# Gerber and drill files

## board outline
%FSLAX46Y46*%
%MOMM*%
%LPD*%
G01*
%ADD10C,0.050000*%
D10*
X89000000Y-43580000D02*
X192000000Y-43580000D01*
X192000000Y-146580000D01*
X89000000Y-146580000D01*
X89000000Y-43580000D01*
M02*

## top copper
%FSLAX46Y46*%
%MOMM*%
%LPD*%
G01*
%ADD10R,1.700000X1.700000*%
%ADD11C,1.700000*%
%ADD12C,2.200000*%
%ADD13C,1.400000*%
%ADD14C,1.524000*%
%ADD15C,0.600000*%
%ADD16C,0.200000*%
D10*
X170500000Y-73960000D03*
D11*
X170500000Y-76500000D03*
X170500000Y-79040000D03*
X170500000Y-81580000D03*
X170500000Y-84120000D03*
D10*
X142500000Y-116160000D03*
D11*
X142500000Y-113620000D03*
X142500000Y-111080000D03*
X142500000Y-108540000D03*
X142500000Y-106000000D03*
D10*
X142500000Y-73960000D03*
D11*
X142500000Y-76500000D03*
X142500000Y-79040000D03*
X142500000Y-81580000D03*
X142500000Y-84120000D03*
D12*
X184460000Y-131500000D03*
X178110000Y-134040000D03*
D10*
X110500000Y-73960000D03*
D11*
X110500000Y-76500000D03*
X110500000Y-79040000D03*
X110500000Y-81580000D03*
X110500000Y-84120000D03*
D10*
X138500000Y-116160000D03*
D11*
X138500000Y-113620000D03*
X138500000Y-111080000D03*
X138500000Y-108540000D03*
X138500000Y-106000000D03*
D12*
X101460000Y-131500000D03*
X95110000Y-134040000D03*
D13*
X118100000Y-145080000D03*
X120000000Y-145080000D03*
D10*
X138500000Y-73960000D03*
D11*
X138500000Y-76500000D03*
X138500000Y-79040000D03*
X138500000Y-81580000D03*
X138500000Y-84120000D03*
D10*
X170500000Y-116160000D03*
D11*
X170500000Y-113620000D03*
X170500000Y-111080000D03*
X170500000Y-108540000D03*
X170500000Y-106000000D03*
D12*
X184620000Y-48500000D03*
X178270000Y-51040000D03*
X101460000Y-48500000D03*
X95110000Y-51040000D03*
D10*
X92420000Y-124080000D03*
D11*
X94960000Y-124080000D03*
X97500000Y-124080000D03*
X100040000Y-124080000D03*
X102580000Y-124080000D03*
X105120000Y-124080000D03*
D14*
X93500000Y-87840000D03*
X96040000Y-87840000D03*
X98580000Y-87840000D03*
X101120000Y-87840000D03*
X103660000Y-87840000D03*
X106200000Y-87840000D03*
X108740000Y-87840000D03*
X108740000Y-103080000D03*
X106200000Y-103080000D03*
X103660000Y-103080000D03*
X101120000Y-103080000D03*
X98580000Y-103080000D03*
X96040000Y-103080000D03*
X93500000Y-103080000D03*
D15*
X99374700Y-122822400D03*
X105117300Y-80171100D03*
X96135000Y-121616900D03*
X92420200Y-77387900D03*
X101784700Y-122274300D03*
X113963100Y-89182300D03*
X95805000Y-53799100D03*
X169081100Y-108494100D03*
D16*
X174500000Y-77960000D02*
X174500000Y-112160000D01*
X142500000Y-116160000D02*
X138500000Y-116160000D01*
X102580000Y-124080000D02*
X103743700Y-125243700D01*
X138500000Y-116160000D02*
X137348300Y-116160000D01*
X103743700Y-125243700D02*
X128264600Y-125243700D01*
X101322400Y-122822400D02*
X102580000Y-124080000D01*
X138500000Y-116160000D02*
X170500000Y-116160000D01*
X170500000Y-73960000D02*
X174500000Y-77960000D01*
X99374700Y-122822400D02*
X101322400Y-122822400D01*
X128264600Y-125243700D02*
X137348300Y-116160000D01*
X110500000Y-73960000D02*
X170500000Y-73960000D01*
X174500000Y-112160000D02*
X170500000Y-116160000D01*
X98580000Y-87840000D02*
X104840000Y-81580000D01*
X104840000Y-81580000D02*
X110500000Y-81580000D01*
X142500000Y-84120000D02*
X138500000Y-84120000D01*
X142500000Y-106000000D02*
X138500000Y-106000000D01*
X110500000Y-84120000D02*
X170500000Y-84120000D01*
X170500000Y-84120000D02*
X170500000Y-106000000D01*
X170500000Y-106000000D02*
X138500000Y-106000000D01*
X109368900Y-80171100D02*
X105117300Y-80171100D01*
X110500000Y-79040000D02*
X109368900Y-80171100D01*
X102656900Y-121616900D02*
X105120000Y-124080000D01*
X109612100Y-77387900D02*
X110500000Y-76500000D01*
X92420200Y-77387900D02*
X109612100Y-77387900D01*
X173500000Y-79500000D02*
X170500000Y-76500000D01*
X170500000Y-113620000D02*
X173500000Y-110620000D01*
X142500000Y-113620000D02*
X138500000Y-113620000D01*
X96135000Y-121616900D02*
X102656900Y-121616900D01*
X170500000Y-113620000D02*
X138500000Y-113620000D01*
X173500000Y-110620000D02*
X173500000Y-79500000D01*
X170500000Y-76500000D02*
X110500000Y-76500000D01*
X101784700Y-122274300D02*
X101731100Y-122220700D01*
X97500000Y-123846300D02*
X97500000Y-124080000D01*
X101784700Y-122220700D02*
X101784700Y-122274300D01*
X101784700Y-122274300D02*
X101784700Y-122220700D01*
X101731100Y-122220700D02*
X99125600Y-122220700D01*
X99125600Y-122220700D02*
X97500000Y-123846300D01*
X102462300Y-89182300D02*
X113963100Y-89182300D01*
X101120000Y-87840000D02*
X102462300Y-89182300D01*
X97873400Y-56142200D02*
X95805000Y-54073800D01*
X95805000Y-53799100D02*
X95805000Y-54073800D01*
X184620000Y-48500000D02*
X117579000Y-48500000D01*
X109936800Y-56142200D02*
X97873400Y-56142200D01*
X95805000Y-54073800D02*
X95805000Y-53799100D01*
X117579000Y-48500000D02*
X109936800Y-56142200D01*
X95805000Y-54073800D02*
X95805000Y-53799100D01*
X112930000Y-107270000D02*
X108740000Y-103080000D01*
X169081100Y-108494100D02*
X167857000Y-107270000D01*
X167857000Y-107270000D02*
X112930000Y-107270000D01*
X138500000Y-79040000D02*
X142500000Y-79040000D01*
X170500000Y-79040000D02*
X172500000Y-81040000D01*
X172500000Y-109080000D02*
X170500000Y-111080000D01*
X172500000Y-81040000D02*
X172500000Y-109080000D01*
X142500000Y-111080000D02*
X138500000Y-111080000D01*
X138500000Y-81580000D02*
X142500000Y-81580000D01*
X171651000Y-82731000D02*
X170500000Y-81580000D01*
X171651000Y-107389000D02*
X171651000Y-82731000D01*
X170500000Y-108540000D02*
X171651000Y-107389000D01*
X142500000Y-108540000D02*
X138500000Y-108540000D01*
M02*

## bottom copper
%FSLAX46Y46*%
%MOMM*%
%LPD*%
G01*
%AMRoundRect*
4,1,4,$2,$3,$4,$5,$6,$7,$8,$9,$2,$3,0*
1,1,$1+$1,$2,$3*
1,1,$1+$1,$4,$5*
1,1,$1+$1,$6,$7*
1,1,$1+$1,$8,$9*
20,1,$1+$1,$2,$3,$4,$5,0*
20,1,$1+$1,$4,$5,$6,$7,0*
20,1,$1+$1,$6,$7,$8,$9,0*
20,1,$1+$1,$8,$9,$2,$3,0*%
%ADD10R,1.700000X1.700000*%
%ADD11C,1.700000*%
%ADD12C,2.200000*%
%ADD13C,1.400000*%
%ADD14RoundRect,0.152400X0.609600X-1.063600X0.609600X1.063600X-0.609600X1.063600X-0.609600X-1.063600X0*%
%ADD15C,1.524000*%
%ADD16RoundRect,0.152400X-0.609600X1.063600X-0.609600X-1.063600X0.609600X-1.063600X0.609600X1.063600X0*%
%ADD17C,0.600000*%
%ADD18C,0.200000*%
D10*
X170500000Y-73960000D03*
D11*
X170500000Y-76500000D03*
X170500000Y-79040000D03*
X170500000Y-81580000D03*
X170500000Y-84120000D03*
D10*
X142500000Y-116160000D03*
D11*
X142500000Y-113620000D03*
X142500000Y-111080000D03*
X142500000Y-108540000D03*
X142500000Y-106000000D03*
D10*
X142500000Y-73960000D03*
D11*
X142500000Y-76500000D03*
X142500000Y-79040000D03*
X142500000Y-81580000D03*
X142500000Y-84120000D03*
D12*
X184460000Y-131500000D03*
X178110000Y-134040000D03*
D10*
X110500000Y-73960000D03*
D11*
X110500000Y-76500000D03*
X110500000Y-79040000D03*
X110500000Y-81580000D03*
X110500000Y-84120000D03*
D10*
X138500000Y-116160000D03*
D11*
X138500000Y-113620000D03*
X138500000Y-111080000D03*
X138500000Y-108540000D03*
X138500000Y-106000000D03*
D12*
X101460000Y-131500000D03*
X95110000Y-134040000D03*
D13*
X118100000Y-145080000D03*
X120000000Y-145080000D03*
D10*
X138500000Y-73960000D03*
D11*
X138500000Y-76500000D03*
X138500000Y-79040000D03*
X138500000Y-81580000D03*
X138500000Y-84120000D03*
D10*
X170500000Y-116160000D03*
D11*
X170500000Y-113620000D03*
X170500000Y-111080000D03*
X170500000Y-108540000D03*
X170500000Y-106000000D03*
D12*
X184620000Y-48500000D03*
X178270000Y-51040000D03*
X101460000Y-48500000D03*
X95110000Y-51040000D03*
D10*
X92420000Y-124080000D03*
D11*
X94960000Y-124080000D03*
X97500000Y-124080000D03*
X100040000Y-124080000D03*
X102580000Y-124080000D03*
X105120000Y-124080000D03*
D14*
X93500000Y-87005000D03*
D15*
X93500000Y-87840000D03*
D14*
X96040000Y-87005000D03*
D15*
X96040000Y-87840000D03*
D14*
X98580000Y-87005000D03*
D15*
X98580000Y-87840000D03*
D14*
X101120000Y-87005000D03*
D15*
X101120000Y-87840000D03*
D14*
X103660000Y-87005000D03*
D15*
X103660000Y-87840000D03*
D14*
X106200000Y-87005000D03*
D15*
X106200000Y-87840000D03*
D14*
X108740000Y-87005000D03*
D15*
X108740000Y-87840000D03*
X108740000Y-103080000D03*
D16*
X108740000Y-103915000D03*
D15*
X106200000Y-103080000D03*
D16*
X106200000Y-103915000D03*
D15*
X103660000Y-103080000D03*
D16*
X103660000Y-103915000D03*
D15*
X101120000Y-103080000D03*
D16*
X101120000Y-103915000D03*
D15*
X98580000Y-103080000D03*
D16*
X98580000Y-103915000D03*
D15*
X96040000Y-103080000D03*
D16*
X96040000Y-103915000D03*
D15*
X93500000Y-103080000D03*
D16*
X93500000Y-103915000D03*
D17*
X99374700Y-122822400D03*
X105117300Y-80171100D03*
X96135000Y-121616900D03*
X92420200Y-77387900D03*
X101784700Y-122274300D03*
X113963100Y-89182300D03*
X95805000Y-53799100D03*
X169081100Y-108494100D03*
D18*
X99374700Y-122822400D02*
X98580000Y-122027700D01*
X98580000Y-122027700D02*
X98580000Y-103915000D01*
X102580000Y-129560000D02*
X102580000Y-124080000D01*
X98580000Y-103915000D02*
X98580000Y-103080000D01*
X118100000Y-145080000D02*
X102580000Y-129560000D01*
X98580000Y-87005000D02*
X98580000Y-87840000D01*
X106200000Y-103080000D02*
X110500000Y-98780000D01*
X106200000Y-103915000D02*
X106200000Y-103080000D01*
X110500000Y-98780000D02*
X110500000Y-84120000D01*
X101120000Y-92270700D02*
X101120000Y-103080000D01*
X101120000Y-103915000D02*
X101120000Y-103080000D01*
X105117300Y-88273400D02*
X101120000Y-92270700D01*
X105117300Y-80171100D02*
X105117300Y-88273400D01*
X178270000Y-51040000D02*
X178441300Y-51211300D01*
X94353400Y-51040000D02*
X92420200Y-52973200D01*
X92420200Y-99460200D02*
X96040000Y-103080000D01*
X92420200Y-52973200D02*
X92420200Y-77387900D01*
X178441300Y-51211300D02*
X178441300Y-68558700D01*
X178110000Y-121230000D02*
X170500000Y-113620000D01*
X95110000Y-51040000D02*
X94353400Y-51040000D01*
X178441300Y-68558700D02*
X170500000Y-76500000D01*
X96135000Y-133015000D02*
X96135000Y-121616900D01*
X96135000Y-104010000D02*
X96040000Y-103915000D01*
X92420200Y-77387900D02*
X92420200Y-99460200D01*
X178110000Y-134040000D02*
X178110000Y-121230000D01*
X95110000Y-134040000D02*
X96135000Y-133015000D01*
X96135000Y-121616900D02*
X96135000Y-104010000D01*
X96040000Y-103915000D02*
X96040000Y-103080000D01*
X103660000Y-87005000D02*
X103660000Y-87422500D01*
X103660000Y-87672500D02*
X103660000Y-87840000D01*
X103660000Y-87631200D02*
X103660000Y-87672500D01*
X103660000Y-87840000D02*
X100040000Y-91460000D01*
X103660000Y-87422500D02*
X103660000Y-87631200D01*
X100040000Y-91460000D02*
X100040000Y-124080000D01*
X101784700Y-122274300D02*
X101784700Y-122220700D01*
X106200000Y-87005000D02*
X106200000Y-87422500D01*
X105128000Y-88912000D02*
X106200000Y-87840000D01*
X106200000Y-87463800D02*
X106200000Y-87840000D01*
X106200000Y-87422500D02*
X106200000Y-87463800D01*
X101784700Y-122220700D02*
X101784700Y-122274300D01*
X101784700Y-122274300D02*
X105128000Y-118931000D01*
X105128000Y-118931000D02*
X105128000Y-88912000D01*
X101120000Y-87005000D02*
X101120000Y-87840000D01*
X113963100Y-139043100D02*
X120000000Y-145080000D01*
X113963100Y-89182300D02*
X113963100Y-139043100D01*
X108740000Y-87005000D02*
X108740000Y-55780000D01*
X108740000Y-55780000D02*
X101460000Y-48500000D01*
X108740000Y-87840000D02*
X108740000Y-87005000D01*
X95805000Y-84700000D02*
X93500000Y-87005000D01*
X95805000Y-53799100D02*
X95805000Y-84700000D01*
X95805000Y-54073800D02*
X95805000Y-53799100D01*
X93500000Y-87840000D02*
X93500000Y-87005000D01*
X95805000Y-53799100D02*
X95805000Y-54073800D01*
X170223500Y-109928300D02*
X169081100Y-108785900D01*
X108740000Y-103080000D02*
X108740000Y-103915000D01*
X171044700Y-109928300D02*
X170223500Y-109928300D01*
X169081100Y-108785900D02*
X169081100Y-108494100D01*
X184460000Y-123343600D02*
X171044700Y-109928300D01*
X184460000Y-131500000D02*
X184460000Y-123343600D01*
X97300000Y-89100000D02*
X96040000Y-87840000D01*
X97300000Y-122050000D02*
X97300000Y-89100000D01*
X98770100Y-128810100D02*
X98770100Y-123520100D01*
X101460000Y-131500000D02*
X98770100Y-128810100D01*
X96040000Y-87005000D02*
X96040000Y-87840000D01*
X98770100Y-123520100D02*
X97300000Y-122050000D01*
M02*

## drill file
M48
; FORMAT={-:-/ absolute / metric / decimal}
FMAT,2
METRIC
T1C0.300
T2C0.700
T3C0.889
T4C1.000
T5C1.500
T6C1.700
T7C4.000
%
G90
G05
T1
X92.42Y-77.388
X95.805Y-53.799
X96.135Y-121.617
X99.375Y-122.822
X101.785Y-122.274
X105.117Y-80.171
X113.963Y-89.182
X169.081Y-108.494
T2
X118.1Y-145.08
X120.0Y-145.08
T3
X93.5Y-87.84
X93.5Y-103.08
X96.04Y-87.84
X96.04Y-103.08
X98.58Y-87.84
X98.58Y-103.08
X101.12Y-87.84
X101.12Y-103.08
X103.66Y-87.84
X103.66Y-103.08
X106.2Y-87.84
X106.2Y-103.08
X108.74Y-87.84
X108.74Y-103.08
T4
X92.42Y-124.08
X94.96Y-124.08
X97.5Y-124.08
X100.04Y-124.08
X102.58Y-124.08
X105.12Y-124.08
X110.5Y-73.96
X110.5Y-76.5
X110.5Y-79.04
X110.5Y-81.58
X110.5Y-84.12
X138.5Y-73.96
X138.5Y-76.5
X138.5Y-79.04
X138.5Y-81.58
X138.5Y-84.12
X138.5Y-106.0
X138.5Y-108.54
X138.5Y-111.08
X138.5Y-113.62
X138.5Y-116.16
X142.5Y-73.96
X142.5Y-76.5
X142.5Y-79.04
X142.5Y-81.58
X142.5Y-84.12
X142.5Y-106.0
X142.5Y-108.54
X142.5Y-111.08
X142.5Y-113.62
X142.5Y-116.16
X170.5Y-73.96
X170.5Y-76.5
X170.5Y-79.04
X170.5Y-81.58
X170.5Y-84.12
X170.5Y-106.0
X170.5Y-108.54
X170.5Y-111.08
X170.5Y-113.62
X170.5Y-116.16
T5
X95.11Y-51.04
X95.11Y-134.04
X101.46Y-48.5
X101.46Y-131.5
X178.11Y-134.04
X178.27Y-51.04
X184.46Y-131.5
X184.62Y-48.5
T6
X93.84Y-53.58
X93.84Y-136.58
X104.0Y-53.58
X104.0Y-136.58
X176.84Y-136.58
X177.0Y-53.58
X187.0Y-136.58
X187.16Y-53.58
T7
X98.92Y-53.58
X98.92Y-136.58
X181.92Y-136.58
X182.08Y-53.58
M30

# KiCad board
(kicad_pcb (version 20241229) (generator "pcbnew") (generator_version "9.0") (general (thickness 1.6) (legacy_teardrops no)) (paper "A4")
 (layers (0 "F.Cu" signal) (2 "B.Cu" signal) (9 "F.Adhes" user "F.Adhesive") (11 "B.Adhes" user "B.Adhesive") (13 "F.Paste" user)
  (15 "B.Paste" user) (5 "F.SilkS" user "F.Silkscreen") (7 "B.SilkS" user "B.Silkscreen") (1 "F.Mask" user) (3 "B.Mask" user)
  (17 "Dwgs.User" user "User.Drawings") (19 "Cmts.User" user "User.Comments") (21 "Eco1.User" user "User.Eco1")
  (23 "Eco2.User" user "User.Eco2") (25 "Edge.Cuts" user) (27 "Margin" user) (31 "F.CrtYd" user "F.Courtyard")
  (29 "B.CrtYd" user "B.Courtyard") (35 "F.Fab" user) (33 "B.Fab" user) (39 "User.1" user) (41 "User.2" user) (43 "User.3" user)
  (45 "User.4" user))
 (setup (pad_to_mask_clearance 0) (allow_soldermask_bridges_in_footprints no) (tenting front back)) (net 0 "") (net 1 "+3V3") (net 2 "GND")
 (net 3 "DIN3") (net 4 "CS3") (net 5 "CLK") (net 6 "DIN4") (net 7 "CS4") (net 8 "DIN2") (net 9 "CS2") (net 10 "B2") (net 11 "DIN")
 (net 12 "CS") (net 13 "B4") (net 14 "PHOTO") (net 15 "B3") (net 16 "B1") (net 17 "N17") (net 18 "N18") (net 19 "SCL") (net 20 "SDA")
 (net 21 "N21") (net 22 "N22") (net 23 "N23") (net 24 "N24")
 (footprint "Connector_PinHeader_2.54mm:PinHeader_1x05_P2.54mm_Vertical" (layer "F.Cu") (at 170.5 73.96)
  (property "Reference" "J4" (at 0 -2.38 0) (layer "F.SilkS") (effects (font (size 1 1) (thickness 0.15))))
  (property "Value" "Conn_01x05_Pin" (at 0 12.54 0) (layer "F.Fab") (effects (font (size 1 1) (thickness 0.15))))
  (pad "1" thru_hole rect (at 0 0) (size 1.7 1.7) (drill 1) (layers "*.Cu" "*.Mask") (remove_unused_layers no) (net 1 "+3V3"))
  (pad "2" thru_hole circle (at 0 2.54) (size 1.7 1.7) (drill 1) (layers "*.Cu" "*.Mask") (remove_unused_layers no) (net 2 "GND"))
  (pad "3" thru_hole circle (at 0 5.08) (size 1.7 1.7) (drill 1) (layers "*.Cu" "*.Mask") (remove_unused_layers no) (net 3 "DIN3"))
  (pad "4" thru_hole circle (at 0 7.62) (size 1.7 1.7) (drill 1) (layers "*.Cu" "*.Mask") (remove_unused_layers no) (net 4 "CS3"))
  (pad "5" thru_hole circle (at 0 10.16) (size 1.7 1.7) (drill 1) (layers "*.Cu" "*.Mask") (remove_unused_layers no) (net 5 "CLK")))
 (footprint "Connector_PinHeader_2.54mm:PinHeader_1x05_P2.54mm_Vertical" (layer "F.Cu") (at 142.5 116.16 180)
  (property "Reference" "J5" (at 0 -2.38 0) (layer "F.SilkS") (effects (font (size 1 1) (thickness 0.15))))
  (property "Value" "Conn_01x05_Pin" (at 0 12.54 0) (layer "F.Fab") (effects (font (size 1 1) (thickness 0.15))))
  (pad "1" thru_hole rect (at 0 0 180) (size 1.7 1.7) (drill 1) (layers "*.Cu" "*.Mask") (remove_unused_layers no) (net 1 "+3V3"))
  (pad "2" thru_hole circle (at 0 2.54 180) (size 1.7 1.7) (drill 1) (layers "*.Cu" "*.Mask") (remove_unused_layers no) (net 2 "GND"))
  (pad "3" thru_hole circle (at 0 5.08 180) (size 1.7 1.7) (drill 1) (layers "*.Cu" "*.Mask") (remove_unused_layers no) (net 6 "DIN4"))
  (pad "4" thru_hole circle (at 0 7.62 180) (size 1.7 1.7) (drill 1) (layers "*.Cu" "*.Mask") (remove_unused_layers no) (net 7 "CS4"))
  (pad "5" thru_hole circle (at 0 10.16 180) (size 1.7 1.7) (drill 1) (layers "*.Cu" "*.Mask") (remove_unused_layers no) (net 5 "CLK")))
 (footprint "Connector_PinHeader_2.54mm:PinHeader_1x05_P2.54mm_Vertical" (layer "F.Cu") (at 142.5 73.96)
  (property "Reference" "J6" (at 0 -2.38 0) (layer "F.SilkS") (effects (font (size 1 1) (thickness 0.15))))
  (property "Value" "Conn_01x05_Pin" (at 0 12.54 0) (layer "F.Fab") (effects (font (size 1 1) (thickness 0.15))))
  (pad "1" thru_hole rect (at 0 0) (size 1.7 1.7) (drill 1) (layers "*.Cu" "*.Mask") (remove_unused_layers no) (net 1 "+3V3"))
  (pad "2" thru_hole circle (at 0 2.54) (size 1.7 1.7) (drill 1) (layers "*.Cu" "*.Mask") (remove_unused_layers no) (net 2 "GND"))
  (pad "3" thru_hole circle (at 0 5.08) (size 1.7 1.7) (drill 1) (layers "*.Cu" "*.Mask") (remove_unused_layers no) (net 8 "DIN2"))
  (pad "4" thru_hole circle (at 0 7.62) (size 1.7 1.7) (drill 1) (layers "*.Cu" "*.Mask") (remove_unused_layers no) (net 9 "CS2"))
  (pad "5" thru_hole circle (at 0 10.16) (size 1.7 1.7) (drill 1) (layers "*.Cu" "*.Mask") (remove_unused_layers no) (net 5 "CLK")))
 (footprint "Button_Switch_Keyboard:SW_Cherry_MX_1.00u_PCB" (layer "F.Cu") (at 184.46 131.5)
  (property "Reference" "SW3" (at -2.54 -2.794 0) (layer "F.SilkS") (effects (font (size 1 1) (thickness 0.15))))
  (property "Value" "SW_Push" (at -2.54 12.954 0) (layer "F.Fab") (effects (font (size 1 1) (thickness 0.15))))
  (pad "" np_thru_hole circle (at -7.62 5.08) (size 1.7 1.7) (drill 1.7) (layers "*.Cu" "*.Mask"))
  (pad "" np_thru_hole circle (at -2.54 5.08) (size 4 4) (drill 4) (layers "*.Cu" "*.Mask"))
  (pad "" np_thru_hole circle (at 2.54 5.08) (size 1.7 1.7) (drill 1.7) (layers "*.Cu" "*.Mask"))
  (pad "1" thru_hole circle (at 0 0) (size 2.2 2.2) (drill 1.5) (layers "*.Cu" "*.Mask") (remove_unused_layers no) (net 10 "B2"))
  (pad "2" thru_hole circle (at -6.35 2.54) (size 2.2 2.2) (drill 1.5) (layers "*.Cu" "*.Mask") (remove_unused_layers no) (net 2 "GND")))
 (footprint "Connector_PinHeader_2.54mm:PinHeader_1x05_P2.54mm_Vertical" (layer "F.Cu") (at 110.5 73.96)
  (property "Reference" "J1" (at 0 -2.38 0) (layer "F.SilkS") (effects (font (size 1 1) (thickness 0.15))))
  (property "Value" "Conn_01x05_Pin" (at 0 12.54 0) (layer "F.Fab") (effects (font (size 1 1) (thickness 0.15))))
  (pad "1" thru_hole rect (at 0 0) (size 1.7 1.7) (drill 1) (layers "*.Cu" "*.Mask") (remove_unused_layers no) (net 1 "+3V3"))
  (pad "2" thru_hole circle (at 0 2.54) (size 1.7 1.7) (drill 1) (layers "*.Cu" "*.Mask") (remove_unused_layers no) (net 2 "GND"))
  (pad "3" thru_hole circle (at 0 5.08) (size 1.7 1.7) (drill 1) (layers "*.Cu" "*.Mask") (remove_unused_layers no) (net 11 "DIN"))
  (pad "4" thru_hole circle (at 0 7.62) (size 1.7 1.7) (drill 1) (layers "*.Cu" "*.Mask") (remove_unused_layers no) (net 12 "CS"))
  (pad "5" thru_hole circle (at 0 10.16) (size 1.7 1.7) (drill 1) (layers "*.Cu" "*.Mask") (remove_unused_layers no) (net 5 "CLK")))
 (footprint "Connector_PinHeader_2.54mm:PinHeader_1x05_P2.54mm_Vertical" (layer "F.Cu") (at 138.5 116.16 180)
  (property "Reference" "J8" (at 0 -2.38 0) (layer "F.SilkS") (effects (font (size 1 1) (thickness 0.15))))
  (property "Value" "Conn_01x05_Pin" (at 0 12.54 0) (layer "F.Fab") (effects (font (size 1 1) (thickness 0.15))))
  (pad "1" thru_hole rect (at 0 0 180) (size 1.7 1.7) (drill 1) (layers "*.Cu" "*.Mask") (remove_unused_layers no) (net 1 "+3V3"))
  (pad "2" thru_hole circle (at 0 2.54 180) (size 1.7 1.7) (drill 1) (layers "*.Cu" "*.Mask") (remove_unused_layers no) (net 2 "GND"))
  (pad "3" thru_hole circle (at 0 5.08 180) (size 1.7 1.7) (drill 1) (layers "*.Cu" "*.Mask") (remove_unused_layers no) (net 6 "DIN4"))
  (pad "4" thru_hole circle (at 0 7.62 180) (size 1.7 1.7) (drill 1) (layers "*.Cu" "*.Mask") (remove_unused_layers no) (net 7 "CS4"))
  (pad "5" thru_hole circle (at 0 10.16 180) (size 1.7 1.7) (drill 1) (layers "*.Cu" "*.Mask") (remove_unused_layers no) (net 5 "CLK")))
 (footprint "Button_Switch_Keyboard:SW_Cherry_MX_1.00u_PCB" (layer "F.Cu") (at 101.46 131.5)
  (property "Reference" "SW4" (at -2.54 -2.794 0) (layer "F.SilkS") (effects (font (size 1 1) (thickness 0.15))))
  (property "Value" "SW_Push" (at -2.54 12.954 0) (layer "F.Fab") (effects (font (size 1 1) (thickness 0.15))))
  (pad "" np_thru_hole circle (at -7.62 5.08) (size 1.7 1.7) (drill 1.7) (layers "*.Cu" "*.Mask"))
  (pad "" np_thru_hole circle (at -2.54 5.08) (size 4 4) (drill 4) (layers "*.Cu" "*.Mask"))
  (pad "" np_thru_hole circle (at 2.54 5.08) (size 1.7 1.7) (drill 1.7) (layers "*.Cu" "*.Mask"))
  (pad "1" thru_hole circle (at 0 0) (size 2.2 2.2) (drill 1.5) (layers "*.Cu" "*.Mask") (remove_unused_layers no) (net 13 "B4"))
  (pad "2" thru_hole circle (at -6.35 2.54) (size 2.2 2.2) (drill 1.5) (layers "*.Cu" "*.Mask") (remove_unused_layers no) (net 2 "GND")))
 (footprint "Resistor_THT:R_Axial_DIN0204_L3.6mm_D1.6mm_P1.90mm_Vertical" (layer "F.Cu") (at 118.1 145.08)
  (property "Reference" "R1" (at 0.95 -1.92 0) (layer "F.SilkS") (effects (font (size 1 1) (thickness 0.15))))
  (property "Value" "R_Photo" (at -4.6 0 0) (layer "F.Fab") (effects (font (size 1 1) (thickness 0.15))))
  (pad "1" thru_hole circle (at 0 0) (size 1.4 1.4) (drill 0.7) (layers "*.Cu" "*.Mask") (remove_unused_layers no) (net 1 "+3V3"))
  (pad "2" thru_hole circle (at 1.9 0) (size 1.4 1.4) (drill 0.7) (layers "*.Cu" "*.Mask") (remove_unused_layers no) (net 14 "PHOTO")))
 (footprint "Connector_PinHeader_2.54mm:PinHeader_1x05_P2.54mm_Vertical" (layer "F.Cu") (at 138.5 73.96)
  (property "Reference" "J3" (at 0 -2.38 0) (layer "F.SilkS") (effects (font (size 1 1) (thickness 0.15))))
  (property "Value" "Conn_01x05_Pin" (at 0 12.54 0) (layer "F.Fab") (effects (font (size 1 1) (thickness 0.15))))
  (pad "1" thru_hole rect (at 0 0) (size 1.7 1.7) (drill 1) (layers "*.Cu" "*.Mask") (remove_unused_layers no) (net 1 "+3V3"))
  (pad "2" thru_hole circle (at 0 2.54) (size 1.7 1.7) (drill 1) (layers "*.Cu" "*.Mask") (remove_unused_layers no) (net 2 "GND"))
  (pad "3" thru_hole circle (at 0 5.08) (size 1.7 1.7) (drill 1) (layers "*.Cu" "*.Mask") (remove_unused_layers no) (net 8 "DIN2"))
  (pad "4" thru_hole circle (at 0 7.62) (size 1.7 1.7) (drill 1) (layers "*.Cu" "*.Mask") (remove_unused_layers no) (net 9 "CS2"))
  (pad "5" thru_hole circle (at 0 10.16) (size 1.7 1.7) (drill 1) (layers "*.Cu" "*.Mask") (remove_unused_layers no) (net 5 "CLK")))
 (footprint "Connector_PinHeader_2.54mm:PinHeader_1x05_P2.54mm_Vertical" (layer "F.Cu") (at 170.5 116.16 180)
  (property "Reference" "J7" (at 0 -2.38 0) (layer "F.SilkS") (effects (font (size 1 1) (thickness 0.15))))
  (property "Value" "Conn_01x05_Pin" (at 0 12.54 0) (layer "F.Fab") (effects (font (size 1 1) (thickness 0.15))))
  (pad "1" thru_hole rect (at 0 0 180) (size 1.7 1.7) (drill 1) (layers "*.Cu" "*.Mask") (remove_unused_layers no) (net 1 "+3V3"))
  (pad "2" thru_hole circle (at 0 2.54 180) (size 1.7 1.7) (drill 1) (layers "*.Cu" "*.Mask") (remove_unused_layers no) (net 2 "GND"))
  (pad "3" thru_hole circle (at 0 5.08 180) (size 1.7 1.7) (drill 1) (layers "*.Cu" "*.Mask") (remove_unused_layers no) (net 3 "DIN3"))
  (pad "4" thru_hole circle (at 0 7.62 180) (size 1.7 1.7) (drill 1) (layers "*.Cu" "*.Mask") (remove_unused_layers no) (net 4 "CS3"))
  (pad "5" thru_hole circle (at 0 10.16 180) (size 1.7 1.7) (drill 1) (layers "*.Cu" "*.Mask") (remove_unused_layers no) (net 5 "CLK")))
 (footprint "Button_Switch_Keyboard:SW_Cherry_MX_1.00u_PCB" (layer "F.Cu") (at 184.62 48.5)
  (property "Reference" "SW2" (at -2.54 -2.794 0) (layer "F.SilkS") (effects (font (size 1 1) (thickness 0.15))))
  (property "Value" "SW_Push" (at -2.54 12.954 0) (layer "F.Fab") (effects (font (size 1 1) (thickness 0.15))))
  (pad "" np_thru_hole circle (at -7.62 5.08) (size 1.7 1.7) (drill 1.7) (layers "*.Cu" "*.Mask"))
  (pad "" np_thru_hole circle (at -2.54 5.08) (size 4 4) (drill 4) (layers "*.Cu" "*.Mask"))
  (pad "" np_thru_hole circle (at 2.54 5.08) (size 1.7 1.7) (drill 1.7) (layers "*.Cu" "*.Mask"))
  (pad "1" thru_hole circle (at 0 0) (size 2.2 2.2) (drill 1.5) (layers "*.Cu" "*.Mask") (remove_unused_layers no) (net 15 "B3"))
  (pad "2" thru_hole circle (at -6.35 2.54) (size 2.2 2.2) (drill 1.5) (layers "*.Cu" "*.Mask") (remove_unused_layers no) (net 2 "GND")))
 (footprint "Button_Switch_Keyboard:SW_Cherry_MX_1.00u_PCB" (layer "F.Cu") (at 101.46 48.5)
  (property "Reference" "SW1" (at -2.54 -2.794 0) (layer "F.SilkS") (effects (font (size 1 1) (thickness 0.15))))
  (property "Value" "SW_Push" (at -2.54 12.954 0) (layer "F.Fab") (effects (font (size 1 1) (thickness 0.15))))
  (pad "" np_thru_hole circle (at -7.62 5.08) (size 1.7 1.7) (drill 1.7) (layers "*.Cu" "*.Mask"))
  (pad "" np_thru_hole circle (at -2.54 5.08) (size 4 4) (drill 4) (layers "*.Cu" "*.Mask"))
  (pad "" np_thru_hole circle (at 2.54 5.08) (size 1.7 1.7) (drill 1.7) (layers "*.Cu" "*.Mask"))
  (pad "1" thru_hole circle (at 0 0) (size 2.2 2.2) (drill 1.5) (layers "*.Cu" "*.Mask") (remove_unused_layers no) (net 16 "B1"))
  (pad "2" thru_hole circle (at -6.35 2.54) (size 2.2 2.2) (drill 1.5) (layers "*.Cu" "*.Mask") (remove_unused_layers no) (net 2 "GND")))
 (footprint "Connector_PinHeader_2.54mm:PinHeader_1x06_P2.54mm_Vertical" (layer "B.Cu") (at 92.42 124.08 -90)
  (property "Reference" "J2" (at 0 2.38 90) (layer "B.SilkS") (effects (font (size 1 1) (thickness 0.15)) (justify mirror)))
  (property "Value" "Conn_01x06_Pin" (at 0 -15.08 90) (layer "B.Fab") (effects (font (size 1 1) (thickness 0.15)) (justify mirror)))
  (pad "1" thru_hole rect (at 0 0 270) (size 1.7 1.7) (drill 1) (layers "*.Cu" "*.Mask") (remove_unused_layers no) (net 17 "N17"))
  (pad "2" thru_hole circle (at 0 -2.54 270) (size 1.7 1.7) (drill 1) (layers "*.Cu" "*.Mask") (remove_unused_layers no) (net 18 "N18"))
  (pad "3" thru_hole circle (at 0 -5.08 270) (size 1.7 1.7) (drill 1) (layers "*.Cu" "*.Mask") (remove_unused_layers no) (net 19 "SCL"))
  (pad "4" thru_hole circle (at 0 -7.62 270) (size 1.7 1.7) (drill 1) (layers "*.Cu" "*.Mask") (remove_unused_layers no) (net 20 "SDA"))
  (pad "5" thru_hole circle (at 0 -10.16 270) (size 1.7 1.7) (drill 1) (layers "*.Cu" "*.Mask") (remove_unused_layers no) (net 1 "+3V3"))
  (pad "6" thru_hole circle (at 0 -12.7 270) (size 1.7 1.7) (drill 1) (layers "*.Cu" "*.Mask") (remove_unused_layers no) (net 2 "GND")))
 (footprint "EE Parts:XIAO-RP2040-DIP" (layer "B.Cu") (at 101.12 95.46 -90)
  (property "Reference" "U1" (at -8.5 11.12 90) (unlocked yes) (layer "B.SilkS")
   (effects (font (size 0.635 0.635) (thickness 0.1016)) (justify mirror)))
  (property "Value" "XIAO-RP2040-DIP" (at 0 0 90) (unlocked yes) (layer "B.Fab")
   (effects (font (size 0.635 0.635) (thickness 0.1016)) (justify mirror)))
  (pad "1" smd roundrect (at -8.455 7.62 90) (size 2.432 1.524) (layers "B.Cu" "B.Mask") (roundrect_rratio 0.1) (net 15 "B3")
   (thermal_bridge_angle 45))
  (pad "1" thru_hole circle (at -7.62 7.62 90) (size 1.524 1.524) (drill 0.889) (layers "*.Cu" "*.Mask") (remove_unused_layers no)
   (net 15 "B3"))
  (pad "2" smd roundrect (at -8.455 5.08 90) (size 2.432 1.524) (layers "B.Cu" "B.Mask") (roundrect_rratio 0.1) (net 13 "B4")
   (thermal_bridge_angle 45))
  (pad "2" thru_hole circle (at -7.62 5.08 90) (size 1.524 1.524) (drill 0.889) (layers "*.Cu" "*.Mask") (remove_unused_layers no)
   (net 13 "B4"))
  (pad "3" smd roundrect (at -8.455 2.54 90) (size 2.432 1.524) (layers "B.Cu" "B.Mask") (roundrect_rratio 0.1) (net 12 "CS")
   (thermal_bridge_angle 45))
  (pad "3" thru_hole circle (at -7.62 2.54 90) (size 1.524 1.524) (drill 0.889) (layers "*.Cu" "*.Mask") (remove_unused_layers no)
   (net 12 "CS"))
  (pad "4" smd roundrect (at -8.455 0 90) (size 2.432 1.524) (layers "B.Cu" "B.Mask") (roundrect_rratio 0.1) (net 14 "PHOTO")
   (thermal_bridge_angle 45))
  (pad "4" thru_hole circle (at -7.62 0 90) (size 1.524 1.524) (drill 0.889) (layers "*.Cu" "*.Mask") (remove_unused_layers no)
   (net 14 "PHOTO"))
  (pad "5" smd roundrect (at -8.455 -2.54 90) (size 2.432 1.524) (layers "B.Cu" "B.Mask") (roundrect_rratio 0.1) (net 20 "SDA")
   (thermal_bridge_angle 45))
  (pad "5" thru_hole circle (at -7.62 -2.54 90) (size 1.524 1.524) (drill 0.889) (layers "*.Cu" "*.Mask") (remove_unused_layers no)
   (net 20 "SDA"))
  (pad "6" smd roundrect (at -8.455 -5.08 90) (size 2.432 1.524) (layers "B.Cu" "B.Mask") (roundrect_rratio 0.1) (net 19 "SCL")
   (thermal_bridge_angle 45))
  (pad "6" thru_hole circle (at -7.62 -5.08 90) (size 1.524 1.524) (drill 0.889) (layers "*.Cu" "*.Mask") (remove_unused_layers no)
   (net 19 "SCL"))
  (pad "7" smd roundrect (at -8.455 -7.62 90) (size 2.432 1.524) (layers "B.Cu" "B.Mask") (roundrect_rratio 0.1) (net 16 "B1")
   (thermal_bridge_angle 45))
  (pad "7" thru_hole circle (at -7.62 -7.62 90) (size 1.524 1.524) (drill 0.889) (layers "*.Cu" "*.Mask") (remove_unused_layers no)
   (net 16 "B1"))
  (pad "8" thru_hole circle (at 7.62 -7.62 270) (size 1.524 1.524) (drill 0.889) (layers "*.Cu" "*.Mask") (remove_unused_layers no)
   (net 10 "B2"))
  (pad "8" smd roundrect (at 8.455 -7.62 270) (size 2.432 1.524) (layers "B.Cu" "B.Mask") (roundrect_rratio 0.1) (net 10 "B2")
   (thermal_bridge_angle 45))
  (pad "9" thru_hole circle (at 7.62 -5.08 270) (size 1.524 1.524) (drill 0.889) (layers "*.Cu" "*.Mask") (remove_unused_layers no)
   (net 5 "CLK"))
  (pad "9" smd roundrect (at 8.455 -5.08 270) (size 2.432 1.524) (layers "B.Cu" "B.Mask") (roundrect_rratio 0.1) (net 5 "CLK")
   (thermal_bridge_angle 45))
  (pad "10" thru_hole circle (at 7.62 -2.54 270) (size 1.524 1.524) (drill 0.889) (layers "*.Cu" "*.Mask") (remove_unused_layers no)
   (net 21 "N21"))
  (pad "10" smd roundrect (at 8.455 -2.54 270) (size 2.432 1.524) (layers "B.Cu" "B.Mask") (roundrect_rratio 0.1) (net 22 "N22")
   (thermal_bridge_angle 45))
  (pad "11" thru_hole circle (at 7.62 0 270) (size 1.524 1.524) (drill 0.889) (layers "*.Cu" "*.Mask") (remove_unused_layers no)
   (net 11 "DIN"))
  (pad "11" smd roundrect (at 8.455 0 270) (size 2.432 1.524) (layers "B.Cu" "B.Mask") (roundrect_rratio 0.1) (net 11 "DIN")
   (thermal_bridge_angle 45))
  (pad "12" thru_hole circle (at 7.62 2.54 270) (size 1.524 1.524) (drill 0.889) (layers "*.Cu" "*.Mask") (remove_unused_layers no)
   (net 1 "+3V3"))
  (pad "12" smd roundrect (at 8.455 2.54 270) (size 2.432 1.524) (layers "B.Cu" "B.Mask") (roundrect_rratio 0.1) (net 1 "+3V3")
   (thermal_bridge_angle 45))
  (pad "13" thru_hole circle (at 7.62 5.08 270) (size 1.524 1.524) (drill 0.889) (layers "*.Cu" "*.Mask") (remove_unused_layers no)
   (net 2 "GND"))
  (pad "13" smd roundrect (at 8.455 5.08 270) (size 2.432 1.524) (layers "B.Cu" "B.Mask") (roundrect_rratio 0.1) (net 2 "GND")
   (thermal_bridge_angle 45))
  (pad "14" thru_hole circle (at 7.62 7.62 270) (size 1.524 1.524) (drill 0.889) (layers "*.Cu" "*.Mask") (remove_unused_layers no)
   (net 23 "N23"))
  (pad "14" smd roundrect (at 8.455 7.62 270) (size 2.432 1.524) (layers "B.Cu" "B.Mask") (roundrect_rratio 0.1) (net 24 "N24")
   (thermal_bridge_angle 45)))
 (gr_rect (start 89 43.58) (end 192 146.58) (stroke (width 0.05) (type default)) (fill no) (layer "Edge.Cuts"))
 (segment (start 174.5 77.96) (end 174.5 112.16) (width 0.2) (layer "F.Cu") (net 1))
 (segment (start 142.5 116.16) (end 138.5 116.16) (width 0.2) (layer "F.Cu") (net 1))
 (segment (start 102.58 124.08) (end 103.7437 125.2437) (width 0.2) (layer "F.Cu") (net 1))
 (segment (start 138.5 116.16) (end 137.3483 116.16) (width 0.2) (layer "F.Cu") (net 1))
 (segment (start 103.7437 125.2437) (end 128.2646 125.2437) (width 0.2) (layer "F.Cu") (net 1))
 (segment (start 101.3224 122.8224) (end 102.58 124.08) (width 0.2) (layer "F.Cu") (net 1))
 (segment (start 138.5 116.16) (end 170.5 116.16) (width 0.2) (layer "F.Cu") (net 1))
 (segment (start 170.5 73.96) (end 174.5 77.96) (width 0.2) (layer "F.Cu") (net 1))
 (segment (start 99.3747 122.8224) (end 101.3224 122.8224) (width 0.2) (layer "F.Cu") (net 1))
 (segment (start 128.2646 125.2437) (end 137.3483 116.16) (width 0.2) (layer "F.Cu") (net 1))
 (segment (start 110.5 73.96) (end 170.5 73.96) (width 0.2) (layer "F.Cu") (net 1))
 (segment (start 174.5 112.16) (end 170.5 116.16) (width 0.2) (layer "F.Cu") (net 1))
 (via (at 99.3747 122.8224) (size 0.6) (drill 0.3) (layers "F.Cu" "B.Cu") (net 1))
 (segment (start 99.3747 122.8224) (end 98.58 122.0277) (width 0.2) (layer "B.Cu") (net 1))
 (segment (start 98.58 122.0277) (end 98.58 103.915) (width 0.2) (layer "B.Cu") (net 1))
 (segment (start 102.58 129.56) (end 102.58 124.08) (width 0.2) (layer "B.Cu") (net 1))
 (segment (start 98.58 103.915) (end 98.58 103.08) (width 0.2) (layer "B.Cu") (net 1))
 (segment (start 118.1 145.08) (end 102.58 129.56) (width 0.2) (layer "B.Cu") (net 1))
 (segment (start 98.58 87.84) (end 104.84 81.58) (width 0.2) (layer "F.Cu") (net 12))
 (segment (start 104.84 81.58) (end 110.5 81.58) (width 0.2) (layer "F.Cu") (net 12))
 (segment (start 98.58 87.005) (end 98.58 87.84) (width 0.2) (layer "B.Cu") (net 12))
 (segment (start 142.5 84.12) (end 138.5 84.12) (width 0.2) (layer "F.Cu") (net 5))
 (segment (start 142.5 106) (end 138.5 106) (width 0.2) (layer "F.Cu") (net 5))
 (segment (start 110.5 84.12) (end 170.5 84.12) (width 0.2) (layer "F.Cu") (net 5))
 (segment (start 170.5 84.12) (end 170.5 106) (width 0.2) (layer "F.Cu") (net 5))
 (segment (start 170.5 106) (end 138.5 106) (width 0.2) (layer "F.Cu") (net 5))
 (segment (start 106.2 103.08) (end 110.5 98.78) (width 0.2) (layer "B.Cu") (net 5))
 (segment (start 106.2 103.915) (end 106.2 103.08) (width 0.2) (layer "B.Cu") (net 5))
 (segment (start 110.5 98.78) (end 110.5 84.12) (width 0.2) (layer "B.Cu") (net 5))
 (segment (start 109.3689 80.1711) (end 105.1173 80.1711) (width 0.2) (layer "F.Cu") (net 11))
 (segment (start 110.5 79.04) (end 109.3689 80.1711) (width 0.2) (layer "F.Cu") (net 11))
 (via (at 105.1173 80.1711) (size 0.6) (drill 0.3) (layers "F.Cu" "B.Cu") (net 11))
 (segment (start 101.12 92.2707) (end 101.12 103.08) (width 0.2) (layer "B.Cu") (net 11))
 (segment (start 101.12 103.915) (end 101.12 103.08) (width 0.2) (layer "B.Cu") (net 11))
 (segment (start 105.1173 88.2734) (end 101.12 92.2707) (width 0.2) (layer "B.Cu") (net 11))
 (segment (start 105.1173 80.1711) (end 105.1173 88.2734) (width 0.2) (layer "B.Cu") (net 11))
 (segment (start 102.6569 121.6169) (end 105.12 124.08) (width 0.2) (layer "F.Cu") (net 2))
 (segment (start 109.6121 77.3879) (end 110.5 76.5) (width 0.2) (layer "F.Cu") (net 2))
 (segment (start 92.4202 77.3879) (end 109.6121 77.3879) (width 0.2) (layer "F.Cu") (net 2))
 (segment (start 173.5 79.5) (end 170.5 76.5) (width 0.2) (layer "F.Cu") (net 2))
 (segment (start 170.5 113.62) (end 173.5 110.62) (width 0.2) (layer "F.Cu") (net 2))
 (segment (start 142.5 113.62) (end 138.5 113.62) (width 0.2) (layer "F.Cu") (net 2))
 (segment (start 96.135 121.6169) (end 102.6569 121.6169) (width 0.2) (layer "F.Cu") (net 2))
 (segment (start 170.5 113.62) (end 138.5 113.62) (width 0.2) (layer "F.Cu") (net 2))
 (segment (start 173.5 110.62) (end 173.5 79.5) (width 0.2) (layer "F.Cu") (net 2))
 (segment (start 170.5 76.5) (end 110.5 76.5) (width 0.2) (layer "F.Cu") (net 2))
 (via (at 96.135 121.6169) (size 0.6) (drill 0.3) (layers "F.Cu" "B.Cu") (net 2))
 (via (at 92.4202 77.3879) (size 0.6) (drill 0.3) (layers "F.Cu" "B.Cu") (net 2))
 (segment (start 178.27 51.04) (end 178.4413 51.2113) (width 0.2) (layer "B.Cu") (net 2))
 (segment (start 94.3534 51.04) (end 92.4202 52.9732) (width 0.2) (layer "B.Cu") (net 2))
 (segment (start 92.4202 99.4602) (end 96.04 103.08) (width 0.2) (layer "B.Cu") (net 2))
 (segment (start 92.4202 52.9732) (end 92.4202 77.3879) (width 0.2) (layer "B.Cu") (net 2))
 (segment (start 178.4413 51.2113) (end 178.4413 68.5587) (width 0.2) (layer "B.Cu") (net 2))
 (segment (start 178.11 121.23) (end 170.5 113.62) (width 0.2) (layer "B.Cu") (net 2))
 (segment (start 95.11 51.04) (end 94.3534 51.04) (width 0.2) (layer "B.Cu") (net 2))
 (segment (start 178.4413 68.5587) (end 170.5 76.5) (width 0.2) (layer "B.Cu") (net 2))
 (segment (start 96.135 133.015) (end 96.135 121.6169) (width 0.2) (layer "B.Cu") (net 2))
 (segment (start 96.135 104.01) (end 96.04 103.915) (width 0.2) (layer "B.Cu") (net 2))
 (segment (start 92.4202 77.3879) (end 92.4202 99.4602) (width 0.2) (layer "B.Cu") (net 2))
 (segment (start 178.11 134.04) (end 178.11 121.23) (width 0.2) (layer "B.Cu") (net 2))
 (segment (start 95.11 134.04) (end 96.135 133.015) (width 0.2) (layer "B.Cu") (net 2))
 (segment (start 96.135 121.6169) (end 96.135 104.01) (width 0.2) (layer "B.Cu") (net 2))
 (segment (start 96.04 103.915) (end 96.04 103.08) (width 0.2) (layer "B.Cu") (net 2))
 (segment (start 103.66 87.005) (end 103.66 87.4225) (width 0.2) (layer "B.Cu") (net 20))
 (segment (start 103.66 87.6725) (end 103.66 87.84) (width 0.2) (layer "B.Cu") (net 20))
 (segment (start 103.66 87.6312) (end 103.66 87.6725) (width 0.2) (layer "B.Cu") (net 20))
 (segment (start 103.66 87.84) (end 100.04 91.46) (width 0.2) (layer "B.Cu") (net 20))
 (segment (start 103.66 87.4225) (end 103.66 87.6312) (width 0.2) (layer "B.Cu") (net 20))
 (segment (start 100.04 91.46) (end 100.04 124.08) (width 0.2) (layer "B.Cu") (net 20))
 (segment (start 101.7847 122.2743) (end 101.7311 122.2207) (width 0.2) (layer "F.Cu") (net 19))
 (segment (start 97.5 123.8463) (end 97.5 124.08) (width 0.2) (layer "F.Cu") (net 19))
 (segment (start 101.7847 122.2207) (end 101.7847 122.2743) (width 0.2) (layer "F.Cu") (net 19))
 (segment (start 101.7847 122.2743) (end 101.7847 122.2207) (width 0.2) (layer "F.Cu") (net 19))
 (segment (start 101.7311 122.2207) (end 99.1256 122.2207) (width 0.2) (layer "F.Cu") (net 19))
 (segment (start 99.1256 122.2207) (end 97.5 123.8463) (width 0.2) (layer "F.Cu") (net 19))
 (via (at 101.7847 122.2743) (size 0.6) (drill 0.3) (layers "F.Cu" "B.Cu") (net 19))
 (segment (start 101.7847 122.2743) (end 101.7847 122.2207) (width 0.2) (layer "B.Cu") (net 19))
 (segment (start 106.2 87.005) (end 106.2 87.4225) (width 0.2) (layer "B.Cu") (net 19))
 (segment (start 105.128 88.912) (end 106.2 87.84) (width 0.2) (layer "B.Cu") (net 19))
 (segment (start 106.2 87.4638) (end 106.2 87.84) (width 0.2) (layer "B.Cu") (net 19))
 (segment (start 106.2 87.4225) (end 106.2 87.4638) (width 0.2) (layer "B.Cu") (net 19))
 (segment (start 101.7847 122.2207) (end 101.7847 122.2743) (width 0.2) (layer "B.Cu") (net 19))
 (segment (start 101.7847 122.2743) (end 105.128 118.931) (width 0.2) (layer "B.Cu") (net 19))
 (segment (start 105.128 118.931) (end 105.128 88.912) (width 0.2) (layer "B.Cu") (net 19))
 (segment (start 102.4623 89.1823) (end 113.9631 89.1823) (width 0.2) (layer "F.Cu") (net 14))
 (segment (start 101.12 87.84) (end 102.4623 89.1823) (width 0.2) (layer "F.Cu") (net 14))
 (via (at 113.9631 89.1823) (size 0.6) (drill 0.3) (layers "F.Cu" "B.Cu") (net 14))
 (segment (start 101.12 87.005) (end 101.12 87.84) (width 0.2) (layer "B.Cu") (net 14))
 (segment (start 113.9631 139.0431) (end 120 145.08) (width 0.2) (layer "B.Cu") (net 14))
 (segment (start 113.9631 89.1823) (end 113.9631 139.0431) (width 0.2) (layer "B.Cu") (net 14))
 (segment (start 108.74 87.005) (end 108.74 55.78) (width 0.2) (layer "B.Cu") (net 16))
 (segment (start 108.74 55.78) (end 101.46 48.5) (width 0.2) (layer "B.Cu") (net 16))
 (segment (start 108.74 87.84) (end 108.74 87.005) (width 0.2) (layer "B.Cu") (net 16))
 (segment (start 97.8734 56.1422) (end 95.805 54.0738) (width 0.2) (layer "F.Cu") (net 15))
 (segment (start 95.805 53.7991) (end 95.805 54.0738) (width 0.2) (layer "F.Cu") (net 15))
 (segment (start 184.62 48.5) (end 117.579 48.5) (width 0.2) (layer "F.Cu") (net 15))
 (segment (start 109.9368 56.1422) (end 97.8734 56.1422) (width 0.2) (layer "F.Cu") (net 15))
 (segment (start 95.805 54.0738) (end 95.805 53.7991) (width 0.2) (layer "F.Cu") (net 15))
 (segment (start 117.579 48.5) (end 109.9368 56.1422) (width 0.2) (layer "F.Cu") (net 15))
 (segment (start 95.805 54.0738) (end 95.805 53.7991) (width 0.2) (layer "F.Cu") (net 15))
 (via (at 95.805 53.7991) (size 0.6) (drill 0.3) (layers "F.Cu" "B.Cu") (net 15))
 (segment (start 95.805 84.7) (end 93.5 87.005) (width 0.2) (layer "B.Cu") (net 15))
 (segment (start 95.805 53.7991) (end 95.805 84.7) (width 0.2) (layer "B.Cu") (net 15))
 (segment (start 95.805 54.0738) (end 95.805 53.7991) (width 0.2) (layer "B.Cu") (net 15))
 (segment (start 93.5 87.84) (end 93.5 87.005) (width 0.2) (layer "B.Cu") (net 15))
 (segment (start 95.805 53.7991) (end 95.805 54.0738) (width 0.2) (layer "B.Cu") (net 15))
 (segment (start 112.93 107.27) (end 108.74 103.08) (width 0.2) (layer "F.Cu") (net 10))
 (segment (start 169.0811 108.4941) (end 167.857 107.27) (width 0.2) (layer "F.Cu") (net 10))
 (segment (start 167.857 107.27) (end 112.93 107.27) (width 0.2) (layer "F.Cu") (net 10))
 (via (at 169.0811 108.4941) (size 0.6) (drill 0.3) (layers "F.Cu" "B.Cu") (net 10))
 (segment (start 170.2235 109.9283) (end 169.0811 108.7859) (width 0.2) (layer "B.Cu") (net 10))
 (segment (start 108.74 103.08) (end 108.74 103.915) (width 0.2) (layer "B.Cu") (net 10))
 (segment (start 171.0447 109.9283) (end 170.2235 109.9283) (width 0.2) (layer "B.Cu") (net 10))
 (segment (start 169.0811 108.7859) (end 169.0811 108.4941) (width 0.2) (layer "B.Cu") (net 10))
 (segment (start 184.46 123.3436) (end 171.0447 109.9283) (width 0.2) (layer "B.Cu") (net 10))
 (segment (start 184.46 131.5) (end 184.46 123.3436) (width 0.2) (layer "B.Cu") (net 10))
 (segment (start 97.3 89.1) (end 96.04 87.84) (width 0.2) (layer "B.Cu") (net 13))
 (segment (start 97.3 122.05) (end 97.3 89.1) (width 0.2) (layer "B.Cu") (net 13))
 (segment (start 98.7701 128.8101) (end 98.7701 123.5201) (width 0.2) (layer "B.Cu") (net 13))
 (segment (start 101.46 131.5) (end 98.7701 128.8101) (width 0.2) (layer "B.Cu") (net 13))
 (segment (start 96.04 87.005) (end 96.04 87.84) (width 0.2) (layer "B.Cu") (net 13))
 (segment (start 98.7701 123.5201) (end 97.3 122.05) (width 0.2) (layer "B.Cu") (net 13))
 (segment (start 138.5 79.04) (end 142.5 79.04) (width 0.2) (layer "F.Cu") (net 8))
 (segment (start 170.5 79.04) (end 172.5 81.04) (width 0.2) (layer "F.Cu") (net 3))
 (segment (start 172.5 109.08) (end 170.5 111.08) (width 0.2) (layer "F.Cu") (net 3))
 (segment (start 172.5 81.04) (end 172.5 109.08) (width 0.2) (layer "F.Cu") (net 3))
 (segment (start 142.5 111.08) (end 138.5 111.08) (width 0.2) (layer "F.Cu") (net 6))
 (segment (start 138.5 81.58) (end 142.5 81.58) (width 0.2) (layer "F.Cu") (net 9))
 (segment (start 171.651 82.731) (end 170.5 81.58) (width 0.2) (layer "F.Cu") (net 4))
 (segment (start 171.651 107.389) (end 171.651 82.731) (width 0.2) (layer "F.Cu") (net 4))
 (segment (start 170.5 108.54) (end 171.651 107.389) (width 0.2) (layer "F.Cu") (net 4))
 (segment (start 142.5 108.54) (end 138.5 108.54) (width 0.2) (layer "F.Cu") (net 7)))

